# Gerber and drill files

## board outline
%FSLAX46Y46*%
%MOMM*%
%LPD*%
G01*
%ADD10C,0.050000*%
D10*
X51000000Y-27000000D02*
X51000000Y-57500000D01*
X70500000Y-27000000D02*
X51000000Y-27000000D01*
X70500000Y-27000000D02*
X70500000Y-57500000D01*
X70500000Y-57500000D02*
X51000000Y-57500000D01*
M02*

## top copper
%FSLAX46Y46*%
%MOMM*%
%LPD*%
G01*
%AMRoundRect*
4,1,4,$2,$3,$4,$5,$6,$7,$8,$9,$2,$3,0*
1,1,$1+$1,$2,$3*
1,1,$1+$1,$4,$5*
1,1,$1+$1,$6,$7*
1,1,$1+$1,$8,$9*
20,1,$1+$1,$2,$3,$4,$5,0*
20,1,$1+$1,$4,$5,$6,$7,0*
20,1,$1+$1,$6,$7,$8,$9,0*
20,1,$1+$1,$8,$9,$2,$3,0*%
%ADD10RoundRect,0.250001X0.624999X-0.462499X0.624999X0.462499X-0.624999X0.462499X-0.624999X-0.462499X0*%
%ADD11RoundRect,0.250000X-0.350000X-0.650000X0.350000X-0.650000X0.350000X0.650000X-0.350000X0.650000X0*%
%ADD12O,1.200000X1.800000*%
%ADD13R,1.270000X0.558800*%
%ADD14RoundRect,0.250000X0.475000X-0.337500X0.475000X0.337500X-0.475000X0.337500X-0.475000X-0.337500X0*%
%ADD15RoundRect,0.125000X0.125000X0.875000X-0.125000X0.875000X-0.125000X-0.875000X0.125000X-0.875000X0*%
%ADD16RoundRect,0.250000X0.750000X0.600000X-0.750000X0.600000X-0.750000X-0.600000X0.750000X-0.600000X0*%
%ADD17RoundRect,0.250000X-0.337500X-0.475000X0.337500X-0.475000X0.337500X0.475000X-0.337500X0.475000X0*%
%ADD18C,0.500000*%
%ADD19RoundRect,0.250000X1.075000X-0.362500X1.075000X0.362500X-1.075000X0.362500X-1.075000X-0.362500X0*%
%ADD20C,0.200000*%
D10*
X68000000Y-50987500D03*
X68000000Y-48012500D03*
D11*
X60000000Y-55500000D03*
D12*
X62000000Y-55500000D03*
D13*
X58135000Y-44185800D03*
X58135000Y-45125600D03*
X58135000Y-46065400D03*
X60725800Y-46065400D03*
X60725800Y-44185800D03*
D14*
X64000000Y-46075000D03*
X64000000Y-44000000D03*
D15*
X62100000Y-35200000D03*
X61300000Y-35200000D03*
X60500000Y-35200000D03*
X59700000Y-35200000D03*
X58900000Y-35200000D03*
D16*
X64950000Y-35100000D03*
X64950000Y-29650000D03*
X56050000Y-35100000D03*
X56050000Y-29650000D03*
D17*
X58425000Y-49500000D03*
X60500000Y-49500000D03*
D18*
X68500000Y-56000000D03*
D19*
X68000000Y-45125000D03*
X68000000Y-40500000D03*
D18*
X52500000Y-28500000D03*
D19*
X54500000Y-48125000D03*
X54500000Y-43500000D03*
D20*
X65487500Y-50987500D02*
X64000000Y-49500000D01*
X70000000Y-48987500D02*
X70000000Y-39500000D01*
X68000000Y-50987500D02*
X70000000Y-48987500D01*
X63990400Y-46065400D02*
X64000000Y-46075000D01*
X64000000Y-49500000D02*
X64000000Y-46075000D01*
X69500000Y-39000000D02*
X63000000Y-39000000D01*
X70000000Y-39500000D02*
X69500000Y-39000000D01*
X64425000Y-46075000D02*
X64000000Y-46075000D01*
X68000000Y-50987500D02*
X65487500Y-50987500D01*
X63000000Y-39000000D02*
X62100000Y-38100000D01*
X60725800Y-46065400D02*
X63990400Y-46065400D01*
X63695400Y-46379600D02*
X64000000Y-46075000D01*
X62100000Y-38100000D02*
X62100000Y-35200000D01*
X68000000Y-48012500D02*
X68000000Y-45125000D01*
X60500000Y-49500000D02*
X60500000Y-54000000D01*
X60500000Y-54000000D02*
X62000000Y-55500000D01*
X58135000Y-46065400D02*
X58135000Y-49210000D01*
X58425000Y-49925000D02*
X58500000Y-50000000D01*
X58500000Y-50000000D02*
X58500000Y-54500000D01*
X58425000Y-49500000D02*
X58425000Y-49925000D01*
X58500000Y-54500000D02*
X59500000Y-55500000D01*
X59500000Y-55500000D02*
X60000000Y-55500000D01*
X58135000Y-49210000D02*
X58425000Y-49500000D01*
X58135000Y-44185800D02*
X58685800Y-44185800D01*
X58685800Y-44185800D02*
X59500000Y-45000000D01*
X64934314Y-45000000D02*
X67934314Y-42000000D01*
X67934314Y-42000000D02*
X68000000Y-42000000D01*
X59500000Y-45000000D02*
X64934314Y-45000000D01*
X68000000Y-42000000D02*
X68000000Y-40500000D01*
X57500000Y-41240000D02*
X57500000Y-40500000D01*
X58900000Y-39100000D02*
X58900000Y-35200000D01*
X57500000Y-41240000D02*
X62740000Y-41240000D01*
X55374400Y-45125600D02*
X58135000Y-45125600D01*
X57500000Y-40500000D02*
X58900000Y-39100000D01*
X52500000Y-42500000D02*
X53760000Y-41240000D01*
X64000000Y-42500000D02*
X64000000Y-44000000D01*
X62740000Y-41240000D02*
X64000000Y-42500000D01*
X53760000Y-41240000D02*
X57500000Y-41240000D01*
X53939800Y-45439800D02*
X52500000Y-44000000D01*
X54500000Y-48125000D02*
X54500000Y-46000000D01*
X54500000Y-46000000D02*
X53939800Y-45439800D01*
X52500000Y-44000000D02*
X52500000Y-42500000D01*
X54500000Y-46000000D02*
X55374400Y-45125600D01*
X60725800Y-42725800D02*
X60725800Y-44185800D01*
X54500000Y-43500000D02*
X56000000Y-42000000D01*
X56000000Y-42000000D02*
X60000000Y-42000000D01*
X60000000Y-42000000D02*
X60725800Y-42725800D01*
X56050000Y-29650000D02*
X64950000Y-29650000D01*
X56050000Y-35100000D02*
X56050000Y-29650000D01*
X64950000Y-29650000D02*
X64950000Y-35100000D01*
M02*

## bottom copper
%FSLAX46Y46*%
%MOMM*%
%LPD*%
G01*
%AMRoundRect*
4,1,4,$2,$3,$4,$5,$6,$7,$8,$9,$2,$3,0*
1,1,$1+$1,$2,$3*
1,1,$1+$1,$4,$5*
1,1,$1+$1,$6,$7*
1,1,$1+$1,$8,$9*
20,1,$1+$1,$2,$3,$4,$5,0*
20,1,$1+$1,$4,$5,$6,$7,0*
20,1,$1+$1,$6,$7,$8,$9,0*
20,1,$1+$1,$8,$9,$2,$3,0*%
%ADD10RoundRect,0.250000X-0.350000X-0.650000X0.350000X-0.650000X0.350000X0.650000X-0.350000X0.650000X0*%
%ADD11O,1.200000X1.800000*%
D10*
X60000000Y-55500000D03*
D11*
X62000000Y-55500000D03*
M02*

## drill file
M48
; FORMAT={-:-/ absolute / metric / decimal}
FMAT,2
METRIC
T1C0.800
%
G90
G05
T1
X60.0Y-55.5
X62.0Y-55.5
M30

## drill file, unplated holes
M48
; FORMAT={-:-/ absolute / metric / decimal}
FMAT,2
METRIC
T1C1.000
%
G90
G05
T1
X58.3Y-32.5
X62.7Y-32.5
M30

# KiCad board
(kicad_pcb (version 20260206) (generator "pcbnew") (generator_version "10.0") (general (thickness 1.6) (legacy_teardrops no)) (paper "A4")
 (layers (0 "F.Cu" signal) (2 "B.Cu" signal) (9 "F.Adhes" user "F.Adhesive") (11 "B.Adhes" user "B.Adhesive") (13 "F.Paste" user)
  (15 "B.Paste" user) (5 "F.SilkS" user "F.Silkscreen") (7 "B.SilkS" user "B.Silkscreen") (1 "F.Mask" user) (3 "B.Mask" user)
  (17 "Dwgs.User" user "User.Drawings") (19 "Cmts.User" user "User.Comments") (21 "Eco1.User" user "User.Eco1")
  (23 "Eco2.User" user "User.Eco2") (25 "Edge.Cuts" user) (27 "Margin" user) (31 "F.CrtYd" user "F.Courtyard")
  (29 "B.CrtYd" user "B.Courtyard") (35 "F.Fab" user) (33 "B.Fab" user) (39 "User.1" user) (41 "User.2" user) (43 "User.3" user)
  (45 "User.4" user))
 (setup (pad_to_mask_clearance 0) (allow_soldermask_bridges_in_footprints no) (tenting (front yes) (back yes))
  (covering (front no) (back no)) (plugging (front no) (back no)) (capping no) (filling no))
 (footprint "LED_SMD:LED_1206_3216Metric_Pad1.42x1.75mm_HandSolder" (layer "F.Cu") (at 68 49.5 90)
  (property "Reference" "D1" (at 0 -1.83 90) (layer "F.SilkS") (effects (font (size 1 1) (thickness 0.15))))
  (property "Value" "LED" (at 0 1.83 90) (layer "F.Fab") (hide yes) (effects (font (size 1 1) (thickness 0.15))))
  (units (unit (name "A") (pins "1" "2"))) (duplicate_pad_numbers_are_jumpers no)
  (pad "1" smd roundrect (at -1.4875 0 90) (size 1.425 1.75) (layers "F.Cu" "F.Mask" "F.Paste") (roundrect_rratio 0.175439)
   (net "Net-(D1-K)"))
  (pad "2" smd roundrect (at 1.4875 0 90) (size 1.425 1.75) (layers "F.Cu" "F.Mask" "F.Paste") (roundrect_rratio 0.175439)
   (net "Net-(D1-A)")))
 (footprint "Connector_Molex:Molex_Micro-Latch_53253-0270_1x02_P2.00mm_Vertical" (layer "F.Cu") (at 60 55.5)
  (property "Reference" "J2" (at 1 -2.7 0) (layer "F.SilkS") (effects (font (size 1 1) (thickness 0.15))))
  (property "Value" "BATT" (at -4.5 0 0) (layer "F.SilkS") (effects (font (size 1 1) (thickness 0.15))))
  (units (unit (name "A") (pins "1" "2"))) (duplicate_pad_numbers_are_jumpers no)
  (pad "1" thru_hole roundrect (at 0 0) (size 1.2 1.8) (drill 0.8) (layers "*.Cu" "*.Mask") (remove_unused_layers no)
   (roundrect_rratio 0.208333) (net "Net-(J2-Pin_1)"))
  (pad "2" thru_hole oval (at 2 0) (size 1.2 1.8) (drill 0.8) (layers "*.Cu" "*.Mask") (remove_unused_layers no) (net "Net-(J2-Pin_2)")))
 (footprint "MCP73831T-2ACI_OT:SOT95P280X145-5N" (layer "F.Cu") (at 59.4304 45.1256)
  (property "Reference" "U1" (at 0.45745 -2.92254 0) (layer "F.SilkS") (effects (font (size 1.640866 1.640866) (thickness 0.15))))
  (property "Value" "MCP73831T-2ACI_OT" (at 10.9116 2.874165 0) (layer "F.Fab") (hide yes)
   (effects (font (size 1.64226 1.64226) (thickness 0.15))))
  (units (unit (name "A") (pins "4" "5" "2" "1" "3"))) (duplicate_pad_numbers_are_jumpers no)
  (pad "1" smd rect (at -1.2954 -0.9398) (size 1.27 0.5588) (layers "F.Cu" "F.Mask" "F.Paste") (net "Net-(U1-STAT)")
   (solder_mask_margin 0.102))
  (pad "2" smd rect (at -1.2954 0) (size 1.27 0.5588) (layers "F.Cu" "F.Mask" "F.Paste") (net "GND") (solder_mask_margin 0.102))
  (pad "3" smd rect (at -1.2954 0.9398) (size 1.27 0.5588) (layers "F.Cu" "F.Mask" "F.Paste") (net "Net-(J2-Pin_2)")
   (solder_mask_margin 0.102))
  (pad "4" smd rect (at 1.2954 0.9398) (size 1.27 0.5588) (layers "F.Cu" "F.Mask" "F.Paste") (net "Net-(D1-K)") (solder_mask_margin 0.102))
  (pad "5" smd rect (at 1.2954 -0.9398) (size 1.27 0.5588) (layers "F.Cu" "F.Mask" "F.Paste") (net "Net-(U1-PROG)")
   (solder_mask_margin 0.102)))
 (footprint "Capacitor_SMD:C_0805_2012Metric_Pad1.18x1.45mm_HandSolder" (layer "F.Cu") (at 64 45.0375 90)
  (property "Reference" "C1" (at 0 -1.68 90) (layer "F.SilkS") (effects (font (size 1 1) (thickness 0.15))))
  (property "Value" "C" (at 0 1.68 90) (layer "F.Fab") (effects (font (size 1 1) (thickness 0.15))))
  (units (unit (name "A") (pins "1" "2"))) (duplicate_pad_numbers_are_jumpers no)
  (pad "1" smd roundrect (at -1.0375 0 90) (size 1.175 1.45) (layers "F.Cu" "F.Mask" "F.Paste") (roundrect_rratio 0.212766)
   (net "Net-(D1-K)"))
  (pad "2" smd roundrect (at 1.0375 0 90) (size 1.175 1.45) (layers "F.Cu" "F.Mask" "F.Paste") (roundrect_rratio 0.212766) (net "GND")))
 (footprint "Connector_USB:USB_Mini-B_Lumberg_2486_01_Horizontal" (layer "F.Cu") (at 60.5 32.5 180)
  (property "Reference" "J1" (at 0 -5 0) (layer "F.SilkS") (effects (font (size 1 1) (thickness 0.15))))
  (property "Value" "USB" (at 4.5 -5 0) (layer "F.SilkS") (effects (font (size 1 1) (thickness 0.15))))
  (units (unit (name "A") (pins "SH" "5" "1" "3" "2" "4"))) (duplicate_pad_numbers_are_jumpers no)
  (pad "" np_thru_hole circle (at -2.2 0 180) (size 1 1) (drill 1) (layers "*.Cu" "*.Mask"))
  (pad "" np_thru_hole circle (at 2.2 0 180) (size 1 1) (drill 1) (layers "*.Cu" "*.Mask"))
  (pad "1" smd roundrect (at -1.6 -2.7 180) (size 0.5 2) (layers "F.Cu" "F.Mask" "F.Paste") (roundrect_rratio 0.25) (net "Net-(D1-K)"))
  (pad "2" smd roundrect (at -0.8 -2.7 180) (size 0.5 2) (layers "F.Cu" "F.Mask" "F.Paste") (roundrect_rratio 0.25)
   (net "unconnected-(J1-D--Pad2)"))
  (pad "3" smd roundrect (at 0 -2.7 180) (size 0.5 2) (layers "F.Cu" "F.Mask" "F.Paste") (roundrect_rratio 0.25)
   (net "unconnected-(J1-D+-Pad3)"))
  (pad "4" smd roundrect (at 0.8 -2.7 180) (size 0.5 2) (layers "F.Cu" "F.Mask" "F.Paste") (roundrect_rratio 0.25)
   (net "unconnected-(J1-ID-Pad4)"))
  (pad "5" smd roundrect (at 1.6 -2.7 180) (size 0.5 2) (layers "F.Cu" "F.Mask" "F.Paste") (roundrect_rratio 0.25) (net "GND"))
  (pad "SH" smd roundrect (at -4.45 -2.6 180) (size 2 1.7) (layers "F.Cu" "F.Mask" "F.Paste") (roundrect_rratio 0.1470588235)
   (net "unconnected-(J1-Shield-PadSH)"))
  (pad "SH" smd roundrect (at -4.45 2.85 180) (size 2 1.7) (layers "F.Cu" "F.Mask" "F.Paste") (roundrect_rratio 0.1470588235)
   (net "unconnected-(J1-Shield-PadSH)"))
  (pad "SH" smd roundrect (at 4.45 -2.6 180) (size 2 1.7) (layers "F.Cu" "F.Mask" "F.Paste") (roundrect_rratio 0.1470588235)
   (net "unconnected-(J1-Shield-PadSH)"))
  (pad "SH" smd roundrect (at 4.45 2.85 180) (size 2 1.7) (layers "F.Cu" "F.Mask" "F.Paste") (roundrect_rratio 0.1470588235)
   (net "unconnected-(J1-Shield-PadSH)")))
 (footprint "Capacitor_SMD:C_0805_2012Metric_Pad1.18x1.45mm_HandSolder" (layer "F.Cu") (at 59.4625 49.5)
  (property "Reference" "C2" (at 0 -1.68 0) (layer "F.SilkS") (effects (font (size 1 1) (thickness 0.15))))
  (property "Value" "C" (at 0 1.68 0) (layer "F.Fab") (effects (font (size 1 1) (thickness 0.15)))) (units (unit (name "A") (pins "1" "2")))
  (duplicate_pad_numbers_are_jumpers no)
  (pad "1" smd roundrect (at -1.0375 0) (size 1.175 1.45) (layers "F.Cu" "F.Mask" "F.Paste") (roundrect_rratio 0.212766)
   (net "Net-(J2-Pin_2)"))
  (pad "2" smd roundrect (at 1.0375 0) (size 1.175 1.45) (layers "F.Cu" "F.Mask" "F.Paste") (roundrect_rratio 0.212766)
   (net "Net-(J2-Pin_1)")))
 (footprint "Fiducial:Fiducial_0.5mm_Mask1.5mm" (layer "F.Cu") (at 68.5 56)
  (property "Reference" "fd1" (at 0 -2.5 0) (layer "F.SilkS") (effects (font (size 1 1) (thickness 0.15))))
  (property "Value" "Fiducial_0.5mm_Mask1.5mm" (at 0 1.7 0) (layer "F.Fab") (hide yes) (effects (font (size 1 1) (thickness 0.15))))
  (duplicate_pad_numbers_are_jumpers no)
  (pad "" smd circle (at 0 0) (size 0.5 0.5) (layers "F.Cu" "F.Mask") (solder_mask_margin 0.5) (clearance 0.6)))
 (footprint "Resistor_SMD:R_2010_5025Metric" (layer "F.Cu") (at 68 42.8125 90)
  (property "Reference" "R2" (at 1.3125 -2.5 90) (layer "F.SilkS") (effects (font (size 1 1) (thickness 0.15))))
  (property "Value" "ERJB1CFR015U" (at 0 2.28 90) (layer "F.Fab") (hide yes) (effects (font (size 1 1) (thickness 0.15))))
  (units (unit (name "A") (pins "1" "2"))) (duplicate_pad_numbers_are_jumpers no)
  (pad "1" smd roundrect (at -2.3125 0 90) (size 1.225 2.65) (layers "F.Cu" "F.Mask" "F.Paste") (roundrect_rratio 0.204082)
   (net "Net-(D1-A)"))
  (pad "2" smd roundrect (at 2.3125 0 90) (size 1.225 2.65) (layers "F.Cu" "F.Mask" "F.Paste") (roundrect_rratio 0.204082)
   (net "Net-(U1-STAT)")))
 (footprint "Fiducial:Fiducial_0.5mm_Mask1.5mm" (layer "F.Cu") (at 52.5 28.5)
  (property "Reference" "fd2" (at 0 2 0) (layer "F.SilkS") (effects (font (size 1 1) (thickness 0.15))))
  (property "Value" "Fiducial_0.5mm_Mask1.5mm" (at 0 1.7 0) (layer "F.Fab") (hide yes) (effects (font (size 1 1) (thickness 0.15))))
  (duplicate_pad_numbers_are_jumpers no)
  (pad "" smd circle (at 0 0) (size 0.5 0.5) (layers "F.Cu" "F.Mask") (solder_mask_margin 0.5) (clearance 0.6)))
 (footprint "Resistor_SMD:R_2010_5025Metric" (layer "F.Cu") (at 54.5 45.8125 90)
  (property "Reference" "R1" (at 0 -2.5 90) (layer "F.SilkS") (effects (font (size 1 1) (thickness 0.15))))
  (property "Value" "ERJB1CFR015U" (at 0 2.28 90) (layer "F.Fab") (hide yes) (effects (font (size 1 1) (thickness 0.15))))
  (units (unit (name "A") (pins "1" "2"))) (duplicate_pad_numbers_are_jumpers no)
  (pad "1" smd roundrect (at -2.3125 0 90) (size 1.225 2.65) (layers "F.Cu" "F.Mask" "F.Paste") (roundrect_rratio 0.204082) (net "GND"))
  (pad "2" smd roundrect (at 2.3125 0 90) (size 1.225 2.65) (layers "F.Cu" "F.Mask" "F.Paste") (roundrect_rratio 0.204082)
   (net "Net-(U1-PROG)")))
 (gr_line (start 51 27) (end 51 57.5) (stroke (width 0.05) (type default)) (layer "Edge.Cuts"))
 (gr_line (start 70.5 27) (end 51 27) (stroke (width 0.05) (type default)) (layer "Edge.Cuts"))
 (gr_line (start 70.5 27) (end 70.5 57.5) (stroke (width 0.05) (type default)) (layer "Edge.Cuts"))
 (gr_line (start 70.5 57.5) (end 51 57.5) (stroke (width 0.05) (type default)) (layer "Edge.Cuts"))
 (segment (start 65.4875 50.9875) (end 64 49.5) (width 0.2) (layer "F.Cu") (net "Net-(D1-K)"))
 (segment (start 70 48.9875) (end 70 39.5) (width 0.2) (layer "F.Cu") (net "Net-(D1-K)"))
 (segment (start 68 50.9875) (end 70 48.9875) (width 0.2) (layer "F.Cu") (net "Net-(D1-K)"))
 (segment (start 63.9904 46.0654) (end 64 46.075) (width 0.2) (layer "F.Cu") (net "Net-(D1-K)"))
 (segment (start 64 49.5) (end 64 46.075) (width 0.2) (layer "F.Cu") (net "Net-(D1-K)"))
 (segment (start 69.5 39) (end 63 39) (width 0.2) (layer "F.Cu") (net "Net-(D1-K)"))
 (segment (start 70 39.5) (end 69.5 39) (width 0.2) (layer "F.Cu") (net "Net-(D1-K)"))
 (segment (start 64.425 46.075) (end 64 46.075) (width 0.2) (layer "F.Cu") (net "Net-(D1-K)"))
 (segment (start 68 50.9875) (end 65.4875 50.9875) (width 0.2) (layer "F.Cu") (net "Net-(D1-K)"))
 (segment (start 63 39) (end 62.1 38.1) (width 0.2) (layer "F.Cu") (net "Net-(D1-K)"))
 (segment (start 60.7258 46.0654) (end 63.9904 46.0654) (width 0.2) (layer "F.Cu") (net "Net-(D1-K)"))
 (segment (start 63.6954 46.3796) (end 64 46.075) (width 0.2) (layer "F.Cu") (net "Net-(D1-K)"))
 (segment (start 62.1 38.1) (end 62.1 35.2) (width 0.2) (layer "F.Cu") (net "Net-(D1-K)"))
 (segment (start 68 48.0125) (end 68 45.125) (width 0.2) (layer "F.Cu") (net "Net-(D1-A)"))
 (segment (start 60.5 49.5) (end 60.5 54) (width 0.2) (layer "F.Cu") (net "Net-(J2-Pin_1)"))
 (segment (start 60.5 54) (end 62 55.5) (width 0.2) (layer "F.Cu") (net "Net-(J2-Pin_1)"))
 (segment (start 58.135 46.0654) (end 58.135 49.21) (width 0.2) (layer "F.Cu") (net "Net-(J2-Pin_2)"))
 (segment (start 58.425 49.925) (end 58.5 50) (width 0.2) (layer "F.Cu") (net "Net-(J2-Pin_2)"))
 (segment (start 58.5 50) (end 58.5 54.5) (width 0.2) (layer "F.Cu") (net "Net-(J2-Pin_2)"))
 (segment (start 58.425 49.5) (end 58.425 49.925) (width 0.2) (layer "F.Cu") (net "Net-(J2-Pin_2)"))
 (segment (start 58.5 54.5) (end 59.5 55.5) (width 0.2) (layer "F.Cu") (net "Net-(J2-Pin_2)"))
 (segment (start 59.5 55.5) (end 60 55.5) (width 0.2) (layer "F.Cu") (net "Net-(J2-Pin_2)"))
 (segment (start 58.135 49.21) (end 58.425 49.5) (width 0.2) (layer "F.Cu") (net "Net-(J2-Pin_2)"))
 (segment (start 58.135 44.1858) (end 58.6858 44.1858) (width 0.2) (layer "F.Cu") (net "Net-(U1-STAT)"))
 (segment (start 58.6858 44.1858) (end 59.5 45) (width 0.2) (layer "F.Cu") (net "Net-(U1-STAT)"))
 (segment (start 64.934314 45) (end 67.934314 42) (width 0.2) (layer "F.Cu") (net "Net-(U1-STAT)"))
 (segment (start 67.934314 42) (end 68 42) (width 0.2) (layer "F.Cu") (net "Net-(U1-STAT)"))
 (segment (start 59.5 45) (end 64.934314 45) (width 0.2) (layer "F.Cu") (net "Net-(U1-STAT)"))
 (segment (start 68 42) (end 68 40.5) (width 0.2) (layer "F.Cu") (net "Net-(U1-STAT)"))
 (segment (start 57.5 41.24) (end 57.5 40.5) (width 0.2) (layer "F.Cu") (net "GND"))
 (segment (start 58.9 39.1) (end 58.9 35.2) (width 0.2) (layer "F.Cu") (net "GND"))
 (segment (start 57.5 41.24) (end 62.74 41.24) (width 0.2) (layer "F.Cu") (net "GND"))
 (segment (start 55.3744 45.1256) (end 58.135 45.1256) (width 0.2) (layer "F.Cu") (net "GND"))
 (segment (start 57.5 40.5) (end 58.9 39.1) (width 0.2) (layer "F.Cu") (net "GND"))
 (segment (start 52.5 42.5) (end 53.76 41.24) (width 0.2) (layer "F.Cu") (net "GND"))
 (segment (start 64 42.5) (end 64 44) (width 0.2) (layer "F.Cu") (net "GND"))
 (segment (start 62.74 41.24) (end 64 42.5) (width 0.2) (layer "F.Cu") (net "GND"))
 (segment (start 53.76 41.24) (end 57.5 41.24) (width 0.2) (layer "F.Cu") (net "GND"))
 (segment (start 53.9398 45.4398) (end 52.5 44) (width 0.2) (layer "F.Cu") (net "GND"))
 (segment (start 54.5 48.125) (end 54.5 46) (width 0.2) (layer "F.Cu") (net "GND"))
 (segment (start 54.5 46) (end 53.9398 45.4398) (width 0.2) (layer "F.Cu") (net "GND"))
 (segment (start 52.5 44) (end 52.5 42.5) (width 0.2) (layer "F.Cu") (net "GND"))
 (segment (start 54.5 46) (end 55.3744 45.1256) (width 0.2) (layer "F.Cu") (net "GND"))
 (segment (start 60.7258 42.7258) (end 60.7258 44.1858) (width 0.2) (layer "F.Cu") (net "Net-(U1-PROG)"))
 (segment (start 54.5 43.5) (end 56 42) (width 0.2) (layer "F.Cu") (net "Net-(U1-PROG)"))
 (segment (start 56 42) (end 60 42) (width 0.2) (layer "F.Cu") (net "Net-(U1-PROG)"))
 (segment (start 60 42) (end 60.7258 42.7258) (width 0.2) (layer "F.Cu") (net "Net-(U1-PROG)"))
 (segment (start 56.05 29.65) (end 64.95 29.65) (width 0.2) (layer "F.Cu") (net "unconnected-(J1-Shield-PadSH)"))
 (segment (start 56.05 35.1) (end 56.05 29.65) (width 0.2) (layer "F.Cu") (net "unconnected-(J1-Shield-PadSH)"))
 (segment (start 64.95 29.65) (end 64.95 35.1) (width 0.2) (layer "F.Cu") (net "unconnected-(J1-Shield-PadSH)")))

